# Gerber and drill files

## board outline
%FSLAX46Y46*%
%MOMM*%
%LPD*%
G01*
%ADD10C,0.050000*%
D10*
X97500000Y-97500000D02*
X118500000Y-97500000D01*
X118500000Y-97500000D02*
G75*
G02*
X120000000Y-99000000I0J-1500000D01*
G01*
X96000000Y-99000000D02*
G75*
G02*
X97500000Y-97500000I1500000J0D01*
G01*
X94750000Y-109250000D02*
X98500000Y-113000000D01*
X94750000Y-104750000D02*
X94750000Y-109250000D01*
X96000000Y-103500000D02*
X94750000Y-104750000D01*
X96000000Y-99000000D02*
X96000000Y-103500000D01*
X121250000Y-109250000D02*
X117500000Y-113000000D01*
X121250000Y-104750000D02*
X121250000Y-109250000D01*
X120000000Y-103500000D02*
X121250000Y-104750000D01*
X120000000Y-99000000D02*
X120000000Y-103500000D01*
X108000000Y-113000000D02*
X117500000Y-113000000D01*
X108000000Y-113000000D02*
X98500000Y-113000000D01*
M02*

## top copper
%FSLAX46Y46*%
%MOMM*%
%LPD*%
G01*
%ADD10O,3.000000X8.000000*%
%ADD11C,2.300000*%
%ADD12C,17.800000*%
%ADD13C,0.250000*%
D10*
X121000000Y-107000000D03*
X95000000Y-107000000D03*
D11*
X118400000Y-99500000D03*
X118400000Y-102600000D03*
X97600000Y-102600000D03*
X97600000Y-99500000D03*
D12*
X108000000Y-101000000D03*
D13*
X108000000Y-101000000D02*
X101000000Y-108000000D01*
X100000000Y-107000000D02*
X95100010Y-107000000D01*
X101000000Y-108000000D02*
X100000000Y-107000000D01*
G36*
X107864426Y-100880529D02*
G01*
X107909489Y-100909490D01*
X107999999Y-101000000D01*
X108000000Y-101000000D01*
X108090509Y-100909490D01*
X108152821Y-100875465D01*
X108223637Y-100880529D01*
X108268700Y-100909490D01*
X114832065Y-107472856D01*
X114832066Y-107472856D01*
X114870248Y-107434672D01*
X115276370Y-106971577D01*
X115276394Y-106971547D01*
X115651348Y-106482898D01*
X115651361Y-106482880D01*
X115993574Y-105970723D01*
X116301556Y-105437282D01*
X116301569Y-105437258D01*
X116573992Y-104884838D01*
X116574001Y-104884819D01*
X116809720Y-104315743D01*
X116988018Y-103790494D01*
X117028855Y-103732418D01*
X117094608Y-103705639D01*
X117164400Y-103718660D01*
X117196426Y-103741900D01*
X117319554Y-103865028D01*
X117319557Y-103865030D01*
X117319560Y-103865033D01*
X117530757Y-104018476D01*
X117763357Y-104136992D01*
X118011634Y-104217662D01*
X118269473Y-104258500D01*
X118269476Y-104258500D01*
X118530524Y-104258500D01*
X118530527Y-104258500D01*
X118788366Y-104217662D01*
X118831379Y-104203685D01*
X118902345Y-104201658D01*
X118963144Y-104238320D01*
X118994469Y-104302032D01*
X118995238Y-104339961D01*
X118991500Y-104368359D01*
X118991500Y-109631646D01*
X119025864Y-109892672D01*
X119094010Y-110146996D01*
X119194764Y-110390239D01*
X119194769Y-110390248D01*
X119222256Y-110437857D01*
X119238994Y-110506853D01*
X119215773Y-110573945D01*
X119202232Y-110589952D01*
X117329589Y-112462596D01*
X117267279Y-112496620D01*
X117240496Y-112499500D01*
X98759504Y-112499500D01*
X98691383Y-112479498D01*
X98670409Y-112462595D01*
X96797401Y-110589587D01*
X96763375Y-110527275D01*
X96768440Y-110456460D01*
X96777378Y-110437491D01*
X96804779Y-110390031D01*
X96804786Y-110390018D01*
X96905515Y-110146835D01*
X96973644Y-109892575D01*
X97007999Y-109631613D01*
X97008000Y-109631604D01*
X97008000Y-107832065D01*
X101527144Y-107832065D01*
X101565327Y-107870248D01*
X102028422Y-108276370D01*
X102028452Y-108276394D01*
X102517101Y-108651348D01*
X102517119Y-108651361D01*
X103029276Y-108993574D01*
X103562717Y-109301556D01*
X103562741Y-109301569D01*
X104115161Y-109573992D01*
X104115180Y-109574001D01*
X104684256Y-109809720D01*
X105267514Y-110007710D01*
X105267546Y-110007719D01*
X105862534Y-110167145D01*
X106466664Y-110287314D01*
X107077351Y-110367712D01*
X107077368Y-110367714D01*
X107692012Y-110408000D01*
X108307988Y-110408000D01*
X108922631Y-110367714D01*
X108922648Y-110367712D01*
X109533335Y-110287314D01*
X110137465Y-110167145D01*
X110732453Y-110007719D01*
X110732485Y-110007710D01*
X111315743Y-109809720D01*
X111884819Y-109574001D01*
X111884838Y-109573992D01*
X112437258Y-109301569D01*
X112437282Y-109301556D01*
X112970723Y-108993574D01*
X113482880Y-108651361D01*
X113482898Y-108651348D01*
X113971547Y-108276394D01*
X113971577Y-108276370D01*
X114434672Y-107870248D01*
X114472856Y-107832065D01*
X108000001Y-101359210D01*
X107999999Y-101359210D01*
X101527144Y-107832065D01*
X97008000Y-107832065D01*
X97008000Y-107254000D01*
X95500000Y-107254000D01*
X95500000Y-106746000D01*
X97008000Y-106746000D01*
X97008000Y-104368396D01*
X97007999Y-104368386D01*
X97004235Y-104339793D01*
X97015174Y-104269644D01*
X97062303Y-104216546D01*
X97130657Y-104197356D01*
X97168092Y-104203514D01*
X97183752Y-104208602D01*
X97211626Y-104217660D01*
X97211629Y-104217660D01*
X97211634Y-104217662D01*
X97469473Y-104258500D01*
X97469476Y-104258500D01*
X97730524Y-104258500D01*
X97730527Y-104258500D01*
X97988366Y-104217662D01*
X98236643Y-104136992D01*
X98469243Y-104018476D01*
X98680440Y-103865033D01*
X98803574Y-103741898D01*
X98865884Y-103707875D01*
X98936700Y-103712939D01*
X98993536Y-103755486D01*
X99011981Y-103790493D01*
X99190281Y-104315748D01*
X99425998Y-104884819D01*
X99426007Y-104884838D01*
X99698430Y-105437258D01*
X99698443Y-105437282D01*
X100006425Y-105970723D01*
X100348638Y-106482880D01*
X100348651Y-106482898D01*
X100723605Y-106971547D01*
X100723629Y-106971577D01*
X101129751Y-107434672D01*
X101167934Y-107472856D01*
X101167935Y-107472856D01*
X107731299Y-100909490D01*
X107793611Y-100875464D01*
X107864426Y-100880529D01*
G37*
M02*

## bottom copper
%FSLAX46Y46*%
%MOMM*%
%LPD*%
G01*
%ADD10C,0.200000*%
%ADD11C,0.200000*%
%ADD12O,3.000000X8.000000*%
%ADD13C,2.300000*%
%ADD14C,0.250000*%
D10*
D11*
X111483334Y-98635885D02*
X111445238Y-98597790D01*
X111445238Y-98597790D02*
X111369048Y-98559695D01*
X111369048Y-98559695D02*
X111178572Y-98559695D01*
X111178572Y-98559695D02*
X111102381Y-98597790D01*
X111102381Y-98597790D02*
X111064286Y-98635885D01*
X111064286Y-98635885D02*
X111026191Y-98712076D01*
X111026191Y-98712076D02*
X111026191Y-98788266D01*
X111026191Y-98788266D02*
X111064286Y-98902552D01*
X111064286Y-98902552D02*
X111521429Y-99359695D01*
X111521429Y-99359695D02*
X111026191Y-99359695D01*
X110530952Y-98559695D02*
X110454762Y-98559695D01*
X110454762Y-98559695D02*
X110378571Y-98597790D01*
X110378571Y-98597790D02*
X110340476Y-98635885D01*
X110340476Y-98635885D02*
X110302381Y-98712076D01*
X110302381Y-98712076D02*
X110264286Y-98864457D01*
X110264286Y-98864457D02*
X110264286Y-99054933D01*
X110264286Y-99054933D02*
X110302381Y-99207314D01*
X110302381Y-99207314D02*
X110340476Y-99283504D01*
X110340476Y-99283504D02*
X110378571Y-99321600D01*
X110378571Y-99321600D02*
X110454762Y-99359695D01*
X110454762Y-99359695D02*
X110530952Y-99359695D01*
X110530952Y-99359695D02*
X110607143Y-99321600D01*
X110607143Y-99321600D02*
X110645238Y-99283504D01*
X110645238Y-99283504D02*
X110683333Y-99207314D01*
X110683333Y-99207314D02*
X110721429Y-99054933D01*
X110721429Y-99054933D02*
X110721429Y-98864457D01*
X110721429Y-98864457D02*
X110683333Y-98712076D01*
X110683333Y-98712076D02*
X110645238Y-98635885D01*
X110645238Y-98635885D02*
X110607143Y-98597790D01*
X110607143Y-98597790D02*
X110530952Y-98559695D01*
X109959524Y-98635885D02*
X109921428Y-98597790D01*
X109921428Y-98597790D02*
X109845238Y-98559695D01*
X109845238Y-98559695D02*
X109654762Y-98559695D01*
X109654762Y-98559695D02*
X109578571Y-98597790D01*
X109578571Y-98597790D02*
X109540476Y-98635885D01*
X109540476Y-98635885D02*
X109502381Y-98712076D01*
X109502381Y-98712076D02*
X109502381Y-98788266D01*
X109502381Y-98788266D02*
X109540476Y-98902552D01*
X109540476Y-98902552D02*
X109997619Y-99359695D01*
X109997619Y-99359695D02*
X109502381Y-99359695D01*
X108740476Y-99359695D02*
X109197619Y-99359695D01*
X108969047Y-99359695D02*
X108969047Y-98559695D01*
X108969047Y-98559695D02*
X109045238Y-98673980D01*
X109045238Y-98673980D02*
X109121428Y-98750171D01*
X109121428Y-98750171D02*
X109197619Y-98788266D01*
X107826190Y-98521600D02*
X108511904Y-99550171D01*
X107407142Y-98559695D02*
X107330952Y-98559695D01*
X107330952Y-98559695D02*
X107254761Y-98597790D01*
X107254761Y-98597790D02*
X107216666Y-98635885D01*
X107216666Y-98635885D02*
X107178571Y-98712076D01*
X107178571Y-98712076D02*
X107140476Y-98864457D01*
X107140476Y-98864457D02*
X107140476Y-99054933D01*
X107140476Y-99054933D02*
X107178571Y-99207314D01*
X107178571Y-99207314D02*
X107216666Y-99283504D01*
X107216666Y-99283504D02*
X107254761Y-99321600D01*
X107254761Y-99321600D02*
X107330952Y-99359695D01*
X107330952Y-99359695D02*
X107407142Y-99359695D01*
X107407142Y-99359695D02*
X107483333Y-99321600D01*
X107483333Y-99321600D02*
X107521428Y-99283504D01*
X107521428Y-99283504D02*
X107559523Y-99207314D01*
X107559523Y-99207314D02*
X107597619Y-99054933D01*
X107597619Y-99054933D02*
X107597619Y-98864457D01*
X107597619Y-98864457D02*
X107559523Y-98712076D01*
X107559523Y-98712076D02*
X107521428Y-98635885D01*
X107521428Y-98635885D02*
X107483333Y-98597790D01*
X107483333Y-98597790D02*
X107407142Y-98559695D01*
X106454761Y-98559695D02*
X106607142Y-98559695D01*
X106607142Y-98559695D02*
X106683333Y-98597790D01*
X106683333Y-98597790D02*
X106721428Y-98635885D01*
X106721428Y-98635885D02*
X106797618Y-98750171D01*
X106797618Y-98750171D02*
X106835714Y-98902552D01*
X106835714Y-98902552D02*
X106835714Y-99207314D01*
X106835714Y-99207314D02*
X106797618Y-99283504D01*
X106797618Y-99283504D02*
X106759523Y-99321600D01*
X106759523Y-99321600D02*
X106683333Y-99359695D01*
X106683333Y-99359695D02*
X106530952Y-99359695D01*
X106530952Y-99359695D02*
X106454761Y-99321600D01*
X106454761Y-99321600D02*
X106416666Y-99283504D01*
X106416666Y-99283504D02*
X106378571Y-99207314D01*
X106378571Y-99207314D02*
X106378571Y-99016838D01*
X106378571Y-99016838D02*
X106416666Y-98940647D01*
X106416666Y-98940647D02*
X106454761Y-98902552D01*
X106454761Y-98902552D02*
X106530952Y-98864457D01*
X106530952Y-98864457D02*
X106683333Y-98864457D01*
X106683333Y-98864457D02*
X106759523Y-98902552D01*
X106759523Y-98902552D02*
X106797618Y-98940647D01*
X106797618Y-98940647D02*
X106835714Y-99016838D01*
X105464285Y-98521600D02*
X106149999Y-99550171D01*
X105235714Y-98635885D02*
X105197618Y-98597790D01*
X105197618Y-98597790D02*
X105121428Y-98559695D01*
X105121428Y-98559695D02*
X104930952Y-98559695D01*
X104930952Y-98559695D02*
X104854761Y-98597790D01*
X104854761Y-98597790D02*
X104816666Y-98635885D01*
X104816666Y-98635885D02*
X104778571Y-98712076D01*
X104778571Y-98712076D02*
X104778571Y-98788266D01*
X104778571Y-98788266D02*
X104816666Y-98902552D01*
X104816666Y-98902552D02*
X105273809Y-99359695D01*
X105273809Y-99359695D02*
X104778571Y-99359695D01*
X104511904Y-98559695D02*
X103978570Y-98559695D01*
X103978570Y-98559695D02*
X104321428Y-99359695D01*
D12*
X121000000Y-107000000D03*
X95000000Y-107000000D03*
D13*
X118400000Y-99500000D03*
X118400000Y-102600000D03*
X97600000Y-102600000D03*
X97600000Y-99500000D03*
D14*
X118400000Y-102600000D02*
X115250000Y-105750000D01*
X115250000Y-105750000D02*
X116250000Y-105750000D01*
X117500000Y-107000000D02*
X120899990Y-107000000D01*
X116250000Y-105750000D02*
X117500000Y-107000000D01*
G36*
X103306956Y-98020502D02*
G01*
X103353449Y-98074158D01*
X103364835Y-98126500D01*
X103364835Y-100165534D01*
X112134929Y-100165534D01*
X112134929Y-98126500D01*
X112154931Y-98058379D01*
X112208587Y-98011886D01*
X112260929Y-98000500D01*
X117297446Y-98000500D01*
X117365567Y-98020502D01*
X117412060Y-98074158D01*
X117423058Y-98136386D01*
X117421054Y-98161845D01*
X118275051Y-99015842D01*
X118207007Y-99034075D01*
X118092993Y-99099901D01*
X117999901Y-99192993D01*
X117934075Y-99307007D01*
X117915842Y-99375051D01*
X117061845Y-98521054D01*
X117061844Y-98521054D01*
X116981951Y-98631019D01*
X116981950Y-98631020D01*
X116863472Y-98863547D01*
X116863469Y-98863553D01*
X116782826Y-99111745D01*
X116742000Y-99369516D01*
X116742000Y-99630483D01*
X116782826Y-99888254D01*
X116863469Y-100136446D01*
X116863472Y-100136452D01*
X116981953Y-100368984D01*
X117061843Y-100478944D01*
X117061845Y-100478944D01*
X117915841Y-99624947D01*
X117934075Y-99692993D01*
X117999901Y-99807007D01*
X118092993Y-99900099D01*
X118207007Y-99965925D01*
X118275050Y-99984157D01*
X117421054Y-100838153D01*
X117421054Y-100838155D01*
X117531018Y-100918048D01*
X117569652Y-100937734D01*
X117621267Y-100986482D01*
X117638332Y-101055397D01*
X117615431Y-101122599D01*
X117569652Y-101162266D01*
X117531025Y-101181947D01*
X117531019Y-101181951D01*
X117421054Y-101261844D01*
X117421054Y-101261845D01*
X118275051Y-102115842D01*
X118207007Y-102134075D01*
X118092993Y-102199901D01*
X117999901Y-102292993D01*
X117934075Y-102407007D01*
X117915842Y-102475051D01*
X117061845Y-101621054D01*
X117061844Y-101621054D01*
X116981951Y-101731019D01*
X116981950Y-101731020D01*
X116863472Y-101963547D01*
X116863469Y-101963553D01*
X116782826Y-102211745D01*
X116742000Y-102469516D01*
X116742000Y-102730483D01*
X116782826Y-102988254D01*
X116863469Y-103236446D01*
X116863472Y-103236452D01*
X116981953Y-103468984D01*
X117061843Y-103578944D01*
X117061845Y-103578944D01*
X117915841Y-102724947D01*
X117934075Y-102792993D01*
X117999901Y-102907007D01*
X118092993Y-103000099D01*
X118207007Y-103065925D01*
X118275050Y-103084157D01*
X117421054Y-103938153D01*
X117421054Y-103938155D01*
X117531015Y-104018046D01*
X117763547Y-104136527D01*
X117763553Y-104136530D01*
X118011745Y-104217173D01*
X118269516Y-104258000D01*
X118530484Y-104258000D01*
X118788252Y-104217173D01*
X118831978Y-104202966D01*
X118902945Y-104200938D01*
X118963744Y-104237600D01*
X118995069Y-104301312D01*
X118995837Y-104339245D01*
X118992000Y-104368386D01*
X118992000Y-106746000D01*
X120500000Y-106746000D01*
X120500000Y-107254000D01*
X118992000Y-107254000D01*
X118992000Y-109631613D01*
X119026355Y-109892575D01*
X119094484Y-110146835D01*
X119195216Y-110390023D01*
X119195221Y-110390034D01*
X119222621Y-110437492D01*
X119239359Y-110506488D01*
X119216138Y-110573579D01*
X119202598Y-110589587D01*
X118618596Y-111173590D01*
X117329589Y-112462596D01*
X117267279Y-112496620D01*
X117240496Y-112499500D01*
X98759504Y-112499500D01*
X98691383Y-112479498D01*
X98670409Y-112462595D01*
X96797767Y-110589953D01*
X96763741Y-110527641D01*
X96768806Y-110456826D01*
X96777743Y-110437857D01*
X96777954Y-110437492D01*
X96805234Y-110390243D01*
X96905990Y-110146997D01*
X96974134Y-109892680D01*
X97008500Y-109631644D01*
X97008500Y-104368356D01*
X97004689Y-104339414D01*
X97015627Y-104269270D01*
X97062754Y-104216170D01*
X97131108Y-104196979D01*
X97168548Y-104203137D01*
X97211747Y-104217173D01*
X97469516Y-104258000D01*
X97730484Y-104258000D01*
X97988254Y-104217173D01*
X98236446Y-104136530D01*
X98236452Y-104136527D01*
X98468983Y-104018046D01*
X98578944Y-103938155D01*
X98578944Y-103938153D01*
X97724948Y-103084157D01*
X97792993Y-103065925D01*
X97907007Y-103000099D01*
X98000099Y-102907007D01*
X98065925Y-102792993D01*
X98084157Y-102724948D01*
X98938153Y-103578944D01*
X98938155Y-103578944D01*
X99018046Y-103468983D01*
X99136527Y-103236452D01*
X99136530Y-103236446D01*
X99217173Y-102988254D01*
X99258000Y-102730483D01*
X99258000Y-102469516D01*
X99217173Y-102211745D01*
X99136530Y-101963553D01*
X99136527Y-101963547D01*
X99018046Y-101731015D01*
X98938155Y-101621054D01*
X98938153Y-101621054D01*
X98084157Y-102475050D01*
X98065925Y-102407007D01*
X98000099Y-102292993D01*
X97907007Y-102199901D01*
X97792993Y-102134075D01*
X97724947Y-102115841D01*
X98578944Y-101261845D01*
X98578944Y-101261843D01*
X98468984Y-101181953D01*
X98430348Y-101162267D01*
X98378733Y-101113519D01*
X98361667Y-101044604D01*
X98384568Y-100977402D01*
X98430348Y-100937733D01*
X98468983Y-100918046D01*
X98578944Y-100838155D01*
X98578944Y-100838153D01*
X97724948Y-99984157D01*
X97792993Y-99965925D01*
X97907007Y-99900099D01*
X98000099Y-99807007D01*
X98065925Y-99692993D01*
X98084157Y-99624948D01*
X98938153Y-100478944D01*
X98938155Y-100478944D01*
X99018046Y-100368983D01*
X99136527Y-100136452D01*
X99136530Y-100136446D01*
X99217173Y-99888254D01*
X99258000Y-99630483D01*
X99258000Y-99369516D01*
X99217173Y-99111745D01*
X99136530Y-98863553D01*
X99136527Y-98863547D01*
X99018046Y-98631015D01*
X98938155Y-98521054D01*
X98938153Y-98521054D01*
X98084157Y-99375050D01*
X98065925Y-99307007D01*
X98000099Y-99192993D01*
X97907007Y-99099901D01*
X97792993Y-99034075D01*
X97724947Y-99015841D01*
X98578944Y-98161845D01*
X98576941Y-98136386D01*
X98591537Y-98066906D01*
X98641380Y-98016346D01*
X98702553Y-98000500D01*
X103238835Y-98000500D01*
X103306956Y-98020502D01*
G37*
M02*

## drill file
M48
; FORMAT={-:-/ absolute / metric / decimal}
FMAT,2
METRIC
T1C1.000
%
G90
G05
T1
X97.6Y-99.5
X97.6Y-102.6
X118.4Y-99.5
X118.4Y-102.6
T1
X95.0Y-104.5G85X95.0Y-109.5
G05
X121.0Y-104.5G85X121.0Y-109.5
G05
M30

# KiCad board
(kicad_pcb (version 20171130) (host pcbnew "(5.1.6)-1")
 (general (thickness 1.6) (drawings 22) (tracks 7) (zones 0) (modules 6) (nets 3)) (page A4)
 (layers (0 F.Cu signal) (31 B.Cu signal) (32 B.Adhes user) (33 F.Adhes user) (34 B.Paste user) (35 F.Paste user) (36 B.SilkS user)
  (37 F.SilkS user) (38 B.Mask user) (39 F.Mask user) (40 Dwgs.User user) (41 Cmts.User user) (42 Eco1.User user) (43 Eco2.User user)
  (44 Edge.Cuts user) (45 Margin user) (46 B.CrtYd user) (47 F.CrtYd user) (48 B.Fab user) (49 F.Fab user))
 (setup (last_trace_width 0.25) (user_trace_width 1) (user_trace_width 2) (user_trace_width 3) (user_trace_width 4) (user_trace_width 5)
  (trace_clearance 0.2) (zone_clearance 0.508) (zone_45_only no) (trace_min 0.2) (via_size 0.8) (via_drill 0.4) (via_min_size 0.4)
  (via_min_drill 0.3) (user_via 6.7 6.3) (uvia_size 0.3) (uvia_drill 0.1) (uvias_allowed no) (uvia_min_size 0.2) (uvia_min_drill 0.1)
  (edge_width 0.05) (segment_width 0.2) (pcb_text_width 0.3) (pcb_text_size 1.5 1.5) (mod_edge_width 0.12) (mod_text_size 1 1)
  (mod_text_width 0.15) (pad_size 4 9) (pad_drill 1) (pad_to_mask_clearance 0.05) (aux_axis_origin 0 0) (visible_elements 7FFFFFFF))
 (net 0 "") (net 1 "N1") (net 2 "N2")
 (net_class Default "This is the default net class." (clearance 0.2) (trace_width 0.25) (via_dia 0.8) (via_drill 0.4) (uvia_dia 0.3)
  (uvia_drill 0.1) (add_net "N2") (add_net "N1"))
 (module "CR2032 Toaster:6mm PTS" (layer F.Cu) (at 121 107)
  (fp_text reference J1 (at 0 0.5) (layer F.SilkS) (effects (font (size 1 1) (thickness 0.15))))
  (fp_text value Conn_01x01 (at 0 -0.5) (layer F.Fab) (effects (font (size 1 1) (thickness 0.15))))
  (pad 1 thru_hole oval (at 0 0) (size 3 8) (drill oval 1 6) (layers *.Cu *.Mask) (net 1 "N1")))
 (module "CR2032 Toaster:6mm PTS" (layer F.Cu) (at 95 107)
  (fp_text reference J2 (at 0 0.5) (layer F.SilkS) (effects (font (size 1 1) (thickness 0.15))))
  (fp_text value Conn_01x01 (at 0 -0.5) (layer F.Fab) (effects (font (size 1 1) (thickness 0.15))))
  (pad 1 thru_hole oval (at 0 0) (size 3 8) (drill oval 1 6) (layers *.Cu *.Mask) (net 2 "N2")))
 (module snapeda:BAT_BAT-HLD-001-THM (layer F.Cu) (at 108 101)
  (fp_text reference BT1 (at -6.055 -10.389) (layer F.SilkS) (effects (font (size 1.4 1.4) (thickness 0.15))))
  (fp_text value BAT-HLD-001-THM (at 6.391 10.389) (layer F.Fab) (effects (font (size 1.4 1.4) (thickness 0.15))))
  (pad P4 thru_hole circle (at 10.4 -1.5) (size 2.3 2.3) (drill 1) (layers *.Cu *.Mask) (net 1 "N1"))
  (pad P3 thru_hole circle (at 10.4 1.6) (size 2.3 2.3) (drill 1) (layers *.Cu *.Mask) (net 1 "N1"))
  (pad P2 thru_hole circle (at -10.4 1.6) (size 2.3 2.3) (drill 1) (layers *.Cu *.Mask) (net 1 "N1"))
  (pad P1 thru_hole circle (at -10.4 -1.5) (size 2.3 2.3) (drill 1) (layers *.Cu *.Mask) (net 1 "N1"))
  (pad N smd circle (at 0 0) (size 17.8 17.8) (layers F.Cu F.Mask) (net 2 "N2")))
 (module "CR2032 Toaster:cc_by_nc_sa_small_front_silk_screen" (layer B.Cu) (at 108 110.75 180)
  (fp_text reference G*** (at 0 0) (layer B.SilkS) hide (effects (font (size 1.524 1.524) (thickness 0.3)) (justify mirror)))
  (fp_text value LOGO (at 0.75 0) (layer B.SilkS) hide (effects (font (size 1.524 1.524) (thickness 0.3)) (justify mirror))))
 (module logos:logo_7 (layer F.Cu) (at 113.75 103)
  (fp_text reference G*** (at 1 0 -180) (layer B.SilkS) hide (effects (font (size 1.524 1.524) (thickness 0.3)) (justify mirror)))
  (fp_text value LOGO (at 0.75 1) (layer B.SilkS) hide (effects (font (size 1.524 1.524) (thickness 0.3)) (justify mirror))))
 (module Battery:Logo (layer F.Cu) (at 0 0)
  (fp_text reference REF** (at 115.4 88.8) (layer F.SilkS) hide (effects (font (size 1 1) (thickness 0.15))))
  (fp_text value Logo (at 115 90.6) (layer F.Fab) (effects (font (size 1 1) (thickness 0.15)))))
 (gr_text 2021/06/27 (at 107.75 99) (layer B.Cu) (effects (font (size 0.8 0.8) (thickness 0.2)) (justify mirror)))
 (gr_line (start 97.5 97.5) (end 118.5 97.5) (layer Edge.Cuts) (width 0.05))
 (gr_arc (start 118.5 99) (end 120 99) (angle -90) (layer Edge.Cuts) (width 0.05))
 (gr_arc (start 97.5 99) (end 97.5 97.5) (angle -90) (layer Edge.Cuts) (width 0.05))
 (gr_line (start 94.75 109.25) (end 98.5 113) (layer Edge.Cuts) (width 0.05))
 (gr_line (start 94.75 104.75) (end 94.75 109.25) (layer Edge.Cuts) (width 0.05))
 (gr_line (start 96 103.5) (end 94.75 104.75) (layer Edge.Cuts) (width 0.05))
 (gr_line (start 96 99) (end 96 103.5) (layer Edge.Cuts) (width 0.05))
 (gr_line (start 121.25 109.25) (end 117.5 113) (layer Edge.Cuts) (width 0.05))
 (gr_line (start 121.25 104.75) (end 121.25 109.25) (layer Edge.Cuts) (width 0.05))
 (gr_line (start 120 103.5) (end 121.25 104.75) (layer Edge.Cuts) (width 0.05))
 (gr_line (start 120 99) (end 120 103.5) (layer Edge.Cuts) (width 0.05))
 (gr_line (start 108 113) (end 117.5 113) (layer Edge.Cuts) (width 0.05))
 (gr_line (start 108 113) (end 98.5 113) (layer Edge.Cuts) (width 0.05))
 (segment (start 118.4 102.6) (end 115.25 105.75) (width 0.25) (layer B.Cu) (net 1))
 (segment (start 115.25 105.75) (end 116.25 105.75) (width 0.25) (layer B.Cu) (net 1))
 (segment (start 117.5 107) (end 120.89999 107) (width 0.25) (layer B.Cu) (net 1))
 (segment (start 116.25 105.75) (end 117.5 107) (width 0.25) (layer B.Cu) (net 1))
 (segment (start 108 101) (end 101 108) (width 0.25) (layer F.Cu) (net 2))
 (segment (start 100 107) (end 95.10001 107) (width 0.25) (layer F.Cu) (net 2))
 (segment (start 101 108) (end 100 107) (width 0.25) (layer F.Cu) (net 2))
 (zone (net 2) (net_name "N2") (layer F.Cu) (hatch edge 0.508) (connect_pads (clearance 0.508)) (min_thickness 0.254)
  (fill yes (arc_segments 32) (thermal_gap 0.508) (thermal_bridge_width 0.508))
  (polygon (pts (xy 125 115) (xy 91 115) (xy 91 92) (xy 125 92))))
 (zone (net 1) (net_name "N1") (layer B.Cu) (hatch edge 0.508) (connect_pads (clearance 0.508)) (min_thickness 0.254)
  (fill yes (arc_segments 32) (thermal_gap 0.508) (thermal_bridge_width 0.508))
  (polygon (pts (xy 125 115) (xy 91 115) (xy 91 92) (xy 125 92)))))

